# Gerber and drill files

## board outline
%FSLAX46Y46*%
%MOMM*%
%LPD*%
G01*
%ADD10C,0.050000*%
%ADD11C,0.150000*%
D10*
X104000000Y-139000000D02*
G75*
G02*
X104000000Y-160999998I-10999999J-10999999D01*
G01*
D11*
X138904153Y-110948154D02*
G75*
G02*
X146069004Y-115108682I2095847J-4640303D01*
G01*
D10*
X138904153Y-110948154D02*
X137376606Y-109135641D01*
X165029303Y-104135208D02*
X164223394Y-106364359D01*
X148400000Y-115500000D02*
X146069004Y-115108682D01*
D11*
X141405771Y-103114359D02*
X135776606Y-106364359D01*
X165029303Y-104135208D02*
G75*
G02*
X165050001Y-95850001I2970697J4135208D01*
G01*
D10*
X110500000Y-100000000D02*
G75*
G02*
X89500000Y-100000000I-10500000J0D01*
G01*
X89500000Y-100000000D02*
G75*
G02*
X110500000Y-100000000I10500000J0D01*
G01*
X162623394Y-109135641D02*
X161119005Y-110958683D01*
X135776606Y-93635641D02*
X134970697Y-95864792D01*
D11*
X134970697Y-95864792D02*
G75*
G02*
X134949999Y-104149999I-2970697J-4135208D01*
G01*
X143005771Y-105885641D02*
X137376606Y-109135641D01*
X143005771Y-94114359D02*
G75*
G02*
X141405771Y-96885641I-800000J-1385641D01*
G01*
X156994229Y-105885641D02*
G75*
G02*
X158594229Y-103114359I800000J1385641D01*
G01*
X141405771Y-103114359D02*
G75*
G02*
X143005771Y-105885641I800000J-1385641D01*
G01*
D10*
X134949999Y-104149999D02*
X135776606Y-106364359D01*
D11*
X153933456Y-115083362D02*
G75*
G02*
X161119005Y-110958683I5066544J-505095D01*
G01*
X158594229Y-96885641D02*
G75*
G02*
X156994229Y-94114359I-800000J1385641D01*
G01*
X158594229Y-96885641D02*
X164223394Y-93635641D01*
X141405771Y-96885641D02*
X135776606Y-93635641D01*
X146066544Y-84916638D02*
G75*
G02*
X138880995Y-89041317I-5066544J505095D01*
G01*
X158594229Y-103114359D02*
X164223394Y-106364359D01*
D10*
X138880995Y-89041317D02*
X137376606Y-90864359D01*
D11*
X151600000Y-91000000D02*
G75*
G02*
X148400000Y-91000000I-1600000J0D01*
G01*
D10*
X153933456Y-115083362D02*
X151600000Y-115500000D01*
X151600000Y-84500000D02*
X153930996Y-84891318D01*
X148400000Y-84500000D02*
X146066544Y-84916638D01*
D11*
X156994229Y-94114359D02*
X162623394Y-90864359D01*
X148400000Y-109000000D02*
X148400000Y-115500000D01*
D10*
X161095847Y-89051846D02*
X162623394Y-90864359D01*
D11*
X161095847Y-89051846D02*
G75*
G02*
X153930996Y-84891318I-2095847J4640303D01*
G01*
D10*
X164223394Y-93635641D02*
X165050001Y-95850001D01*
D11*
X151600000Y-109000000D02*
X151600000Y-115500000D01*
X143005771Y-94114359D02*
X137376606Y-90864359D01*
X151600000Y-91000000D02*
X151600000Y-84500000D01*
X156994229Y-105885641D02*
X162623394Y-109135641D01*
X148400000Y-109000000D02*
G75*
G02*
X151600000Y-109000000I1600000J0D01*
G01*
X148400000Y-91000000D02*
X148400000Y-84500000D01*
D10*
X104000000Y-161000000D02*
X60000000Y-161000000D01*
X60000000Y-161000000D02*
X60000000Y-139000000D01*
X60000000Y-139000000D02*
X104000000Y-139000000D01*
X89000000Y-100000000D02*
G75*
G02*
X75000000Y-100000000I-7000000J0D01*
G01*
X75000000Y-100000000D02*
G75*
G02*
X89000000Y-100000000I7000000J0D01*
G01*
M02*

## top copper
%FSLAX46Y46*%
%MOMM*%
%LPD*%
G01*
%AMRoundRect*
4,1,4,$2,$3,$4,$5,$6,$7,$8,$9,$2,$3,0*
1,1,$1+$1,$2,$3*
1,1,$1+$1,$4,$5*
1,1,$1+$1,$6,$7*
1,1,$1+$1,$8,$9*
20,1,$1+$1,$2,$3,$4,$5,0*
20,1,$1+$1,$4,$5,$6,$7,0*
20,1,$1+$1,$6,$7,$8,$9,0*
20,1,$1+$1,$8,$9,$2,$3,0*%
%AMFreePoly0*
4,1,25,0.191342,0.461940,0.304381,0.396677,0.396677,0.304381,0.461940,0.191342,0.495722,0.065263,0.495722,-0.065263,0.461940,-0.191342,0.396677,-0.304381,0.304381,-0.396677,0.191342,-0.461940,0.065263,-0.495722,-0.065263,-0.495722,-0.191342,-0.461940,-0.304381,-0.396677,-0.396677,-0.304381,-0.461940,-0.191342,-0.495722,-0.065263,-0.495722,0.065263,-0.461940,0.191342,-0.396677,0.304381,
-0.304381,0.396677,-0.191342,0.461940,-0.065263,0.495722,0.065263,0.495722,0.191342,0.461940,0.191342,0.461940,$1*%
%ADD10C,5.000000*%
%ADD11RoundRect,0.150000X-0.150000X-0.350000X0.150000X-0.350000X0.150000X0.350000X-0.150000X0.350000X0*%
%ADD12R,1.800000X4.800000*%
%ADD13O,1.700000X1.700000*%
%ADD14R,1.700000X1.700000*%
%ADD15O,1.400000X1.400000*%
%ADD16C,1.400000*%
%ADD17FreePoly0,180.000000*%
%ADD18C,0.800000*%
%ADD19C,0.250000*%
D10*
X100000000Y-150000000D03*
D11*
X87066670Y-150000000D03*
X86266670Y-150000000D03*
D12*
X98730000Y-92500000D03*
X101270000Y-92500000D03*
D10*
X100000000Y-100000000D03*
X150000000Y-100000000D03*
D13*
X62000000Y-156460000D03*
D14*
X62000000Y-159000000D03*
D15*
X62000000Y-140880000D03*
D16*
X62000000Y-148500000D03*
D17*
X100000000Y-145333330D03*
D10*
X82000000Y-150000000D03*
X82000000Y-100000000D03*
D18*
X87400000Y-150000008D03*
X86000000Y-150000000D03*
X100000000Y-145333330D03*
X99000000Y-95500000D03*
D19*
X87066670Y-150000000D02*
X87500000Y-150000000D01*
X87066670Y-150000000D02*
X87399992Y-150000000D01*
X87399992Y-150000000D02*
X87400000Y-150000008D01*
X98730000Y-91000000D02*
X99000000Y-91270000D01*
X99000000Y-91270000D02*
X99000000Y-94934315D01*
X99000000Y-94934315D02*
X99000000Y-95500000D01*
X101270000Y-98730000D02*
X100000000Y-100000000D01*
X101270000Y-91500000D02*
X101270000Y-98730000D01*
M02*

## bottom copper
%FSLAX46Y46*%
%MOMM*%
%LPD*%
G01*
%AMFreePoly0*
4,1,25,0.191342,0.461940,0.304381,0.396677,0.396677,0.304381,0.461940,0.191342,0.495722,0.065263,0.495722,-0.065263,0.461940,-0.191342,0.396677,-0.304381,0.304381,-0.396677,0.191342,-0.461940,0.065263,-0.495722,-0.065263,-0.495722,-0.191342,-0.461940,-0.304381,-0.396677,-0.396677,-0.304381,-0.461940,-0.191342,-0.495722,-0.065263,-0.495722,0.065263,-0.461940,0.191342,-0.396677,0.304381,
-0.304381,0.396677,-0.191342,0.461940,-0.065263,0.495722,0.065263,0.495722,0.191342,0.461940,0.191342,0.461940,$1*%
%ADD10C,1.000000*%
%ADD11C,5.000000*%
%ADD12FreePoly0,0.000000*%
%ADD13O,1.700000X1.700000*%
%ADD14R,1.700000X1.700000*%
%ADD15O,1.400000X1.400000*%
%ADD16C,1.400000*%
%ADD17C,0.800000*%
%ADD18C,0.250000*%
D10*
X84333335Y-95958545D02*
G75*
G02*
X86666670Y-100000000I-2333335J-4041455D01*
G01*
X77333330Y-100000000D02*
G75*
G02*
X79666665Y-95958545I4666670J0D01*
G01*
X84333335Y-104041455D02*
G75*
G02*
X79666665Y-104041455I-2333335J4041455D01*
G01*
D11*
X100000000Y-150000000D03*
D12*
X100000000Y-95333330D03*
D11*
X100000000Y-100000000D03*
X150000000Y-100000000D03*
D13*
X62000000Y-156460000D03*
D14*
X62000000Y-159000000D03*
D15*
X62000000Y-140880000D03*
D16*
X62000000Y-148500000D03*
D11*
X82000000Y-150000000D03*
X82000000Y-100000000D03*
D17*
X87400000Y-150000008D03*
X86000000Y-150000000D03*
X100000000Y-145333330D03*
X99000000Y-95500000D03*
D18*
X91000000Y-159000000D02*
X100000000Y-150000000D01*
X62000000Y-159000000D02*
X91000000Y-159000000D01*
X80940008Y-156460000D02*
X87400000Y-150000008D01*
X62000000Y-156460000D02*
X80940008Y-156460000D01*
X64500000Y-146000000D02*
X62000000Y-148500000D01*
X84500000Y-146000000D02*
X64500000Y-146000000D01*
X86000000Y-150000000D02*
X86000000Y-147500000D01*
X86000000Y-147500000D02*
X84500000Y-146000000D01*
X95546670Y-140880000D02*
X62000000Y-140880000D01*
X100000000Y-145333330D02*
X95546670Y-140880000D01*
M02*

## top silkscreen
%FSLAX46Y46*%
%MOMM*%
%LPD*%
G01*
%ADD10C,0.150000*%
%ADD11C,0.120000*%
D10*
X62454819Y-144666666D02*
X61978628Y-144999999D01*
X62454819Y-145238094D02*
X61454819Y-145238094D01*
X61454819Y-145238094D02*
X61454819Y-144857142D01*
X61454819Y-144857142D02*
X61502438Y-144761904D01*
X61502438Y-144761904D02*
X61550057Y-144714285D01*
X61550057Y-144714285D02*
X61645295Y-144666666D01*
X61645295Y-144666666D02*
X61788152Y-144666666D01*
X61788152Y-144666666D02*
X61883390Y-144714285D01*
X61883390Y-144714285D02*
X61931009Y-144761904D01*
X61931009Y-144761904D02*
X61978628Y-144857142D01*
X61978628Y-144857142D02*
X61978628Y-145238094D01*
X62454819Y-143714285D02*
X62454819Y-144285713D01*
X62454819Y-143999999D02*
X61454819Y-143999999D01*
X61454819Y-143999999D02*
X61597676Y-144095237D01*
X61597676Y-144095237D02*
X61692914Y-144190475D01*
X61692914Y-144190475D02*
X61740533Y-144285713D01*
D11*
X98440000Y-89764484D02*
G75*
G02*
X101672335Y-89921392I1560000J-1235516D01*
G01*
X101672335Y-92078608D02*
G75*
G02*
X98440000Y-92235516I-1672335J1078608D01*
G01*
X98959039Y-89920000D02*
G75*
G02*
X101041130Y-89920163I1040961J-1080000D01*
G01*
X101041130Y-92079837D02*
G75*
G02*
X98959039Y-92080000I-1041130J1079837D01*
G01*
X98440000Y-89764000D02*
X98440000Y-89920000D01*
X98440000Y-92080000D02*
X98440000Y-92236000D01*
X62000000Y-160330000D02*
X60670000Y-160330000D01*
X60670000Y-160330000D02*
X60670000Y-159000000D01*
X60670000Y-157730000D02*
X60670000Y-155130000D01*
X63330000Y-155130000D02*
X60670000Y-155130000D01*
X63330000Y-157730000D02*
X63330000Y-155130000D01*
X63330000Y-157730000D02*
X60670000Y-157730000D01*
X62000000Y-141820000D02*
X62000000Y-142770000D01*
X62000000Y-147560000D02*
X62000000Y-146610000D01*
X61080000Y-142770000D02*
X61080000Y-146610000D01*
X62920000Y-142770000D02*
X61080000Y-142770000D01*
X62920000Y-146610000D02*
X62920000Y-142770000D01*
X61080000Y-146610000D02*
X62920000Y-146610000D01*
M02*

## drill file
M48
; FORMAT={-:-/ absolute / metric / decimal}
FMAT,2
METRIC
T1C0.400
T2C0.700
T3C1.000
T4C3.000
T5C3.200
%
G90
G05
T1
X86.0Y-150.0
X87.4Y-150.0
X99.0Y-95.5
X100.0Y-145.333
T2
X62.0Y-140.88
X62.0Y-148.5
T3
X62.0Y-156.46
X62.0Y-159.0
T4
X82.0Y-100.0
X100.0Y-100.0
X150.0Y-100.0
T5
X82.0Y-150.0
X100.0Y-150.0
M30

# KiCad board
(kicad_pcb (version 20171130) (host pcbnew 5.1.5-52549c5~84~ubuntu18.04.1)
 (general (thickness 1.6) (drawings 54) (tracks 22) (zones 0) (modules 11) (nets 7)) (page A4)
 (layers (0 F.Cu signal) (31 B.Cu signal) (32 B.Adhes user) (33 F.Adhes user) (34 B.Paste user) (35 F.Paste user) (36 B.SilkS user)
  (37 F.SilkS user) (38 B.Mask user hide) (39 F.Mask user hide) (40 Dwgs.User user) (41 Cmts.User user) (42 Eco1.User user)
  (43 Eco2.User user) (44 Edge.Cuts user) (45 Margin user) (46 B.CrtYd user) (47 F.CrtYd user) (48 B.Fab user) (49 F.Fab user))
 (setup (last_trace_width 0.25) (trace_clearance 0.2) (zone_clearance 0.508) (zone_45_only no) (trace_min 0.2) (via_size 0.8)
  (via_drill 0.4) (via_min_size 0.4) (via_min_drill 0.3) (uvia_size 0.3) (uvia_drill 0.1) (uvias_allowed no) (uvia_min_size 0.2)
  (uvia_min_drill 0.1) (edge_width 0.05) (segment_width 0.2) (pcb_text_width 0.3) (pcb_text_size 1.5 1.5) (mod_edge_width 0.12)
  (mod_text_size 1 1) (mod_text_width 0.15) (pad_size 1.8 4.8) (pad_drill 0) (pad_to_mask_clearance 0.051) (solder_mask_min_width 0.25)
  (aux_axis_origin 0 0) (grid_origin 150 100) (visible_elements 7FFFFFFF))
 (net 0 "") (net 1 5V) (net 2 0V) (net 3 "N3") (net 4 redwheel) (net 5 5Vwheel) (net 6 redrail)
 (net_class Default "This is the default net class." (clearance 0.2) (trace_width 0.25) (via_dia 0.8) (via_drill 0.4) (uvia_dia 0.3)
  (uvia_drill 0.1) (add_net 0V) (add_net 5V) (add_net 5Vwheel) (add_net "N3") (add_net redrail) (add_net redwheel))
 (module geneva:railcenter (layer F.Cu) (at 100 150)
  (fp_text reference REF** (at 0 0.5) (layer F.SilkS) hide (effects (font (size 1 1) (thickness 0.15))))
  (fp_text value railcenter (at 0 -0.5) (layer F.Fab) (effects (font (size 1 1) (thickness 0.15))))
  (pad 1 thru_hole circle (at 0 0) (size 5 5) (drill 3.2) (layers *.Cu *.Mask) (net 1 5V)))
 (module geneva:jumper (layer F.Cu) (at 86.66667 150)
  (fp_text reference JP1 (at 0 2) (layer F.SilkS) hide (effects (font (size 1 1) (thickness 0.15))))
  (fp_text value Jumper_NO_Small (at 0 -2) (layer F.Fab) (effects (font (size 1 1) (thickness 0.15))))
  (pad 2 smd roundrect (at 0.4 0) (size 0.6 1) (layers F.Cu F.Mask) (roundrect_rratio 0.25) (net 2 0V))
  (pad 1 smd roundrect (at -0.4 0) (size 0.6 1) (layers F.Cu F.Mask) (roundrect_rratio 0.25) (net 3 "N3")))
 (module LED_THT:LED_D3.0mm (layer F.Cu) (at 100 91)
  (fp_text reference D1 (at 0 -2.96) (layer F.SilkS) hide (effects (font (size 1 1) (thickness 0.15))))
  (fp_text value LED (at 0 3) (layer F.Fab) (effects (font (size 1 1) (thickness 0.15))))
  (fp_arc (start 0 0) (end -1.56 -1.235516) (angle 108.8) (layer F.SilkS) (width 0.12))
  (fp_arc (start 0 0) (end -1.56 1.235516) (angle -108.8) (layer F.SilkS) (width 0.12))
  (fp_arc (start 0 0) (end -1.040961 -1.08) (angle 87.9) (layer F.SilkS) (width 0.12))
  (fp_arc (start 0 0) (end -1.040961 1.08) (angle -87.9) (layer F.SilkS) (width 0.12))
  (fp_line (start -1.56 -1.236) (end -1.56 -1.08) (layer F.SilkS) (width 0.12))
  (fp_line (start -1.56 1.08) (end -1.56 1.236) (layer F.SilkS) (width 0.12))
  (pad 1 smd rect (at -1.27 1.5) (size 1.8 4.8) (layers F.Cu F.Paste F.Mask) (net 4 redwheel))
  (pad 2 smd rect (at 1.27 1.5) (size 1.8 4.8) (layers F.Cu F.Paste F.Mask) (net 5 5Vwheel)))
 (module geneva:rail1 (layer B.Cu) (at 100 100)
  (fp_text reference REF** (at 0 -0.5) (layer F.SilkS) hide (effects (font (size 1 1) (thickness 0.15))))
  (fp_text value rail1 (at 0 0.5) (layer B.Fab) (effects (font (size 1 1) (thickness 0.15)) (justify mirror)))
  (pad 1 smd custom (at 0 -4.66667) (size 1 1) (layers B.Cu B.Mask) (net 4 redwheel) (zone_connect 0)
   (options (clearance outline) (anchor circle)) (primitives)))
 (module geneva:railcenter (layer F.Cu) (at 100 100)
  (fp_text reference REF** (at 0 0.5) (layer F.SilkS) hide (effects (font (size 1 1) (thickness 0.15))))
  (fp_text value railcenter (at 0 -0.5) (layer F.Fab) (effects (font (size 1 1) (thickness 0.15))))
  (pad 1 thru_hole circle (at 0 0) (size 5 5) (drill 3) (layers *.Cu *.Mask) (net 5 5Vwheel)))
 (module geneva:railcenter (layer F.Cu) (at 150 100)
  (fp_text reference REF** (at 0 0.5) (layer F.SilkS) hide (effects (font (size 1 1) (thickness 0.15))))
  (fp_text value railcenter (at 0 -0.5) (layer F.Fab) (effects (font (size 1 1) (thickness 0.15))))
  (pad 1 thru_hole circle (at 0 0) (size 5 5) (drill 3) (layers *.Cu *.Mask)))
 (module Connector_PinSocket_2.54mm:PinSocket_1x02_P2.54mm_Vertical (layer F.Cu) (at 62 159 180)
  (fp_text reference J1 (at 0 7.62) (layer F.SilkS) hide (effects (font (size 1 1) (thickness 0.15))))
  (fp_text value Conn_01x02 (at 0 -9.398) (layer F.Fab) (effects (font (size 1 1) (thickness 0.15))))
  (fp_line (start 0 -1.33) (end 1.33 -1.33) (layer F.SilkS) (width 0.12))
  (fp_line (start 1.33 -1.33) (end 1.33 0) (layer F.SilkS) (width 0.12))
  (fp_line (start 1.33 1.27) (end 1.33 3.87) (layer F.SilkS) (width 0.12))
  (fp_line (start -1.33 3.87) (end 1.33 3.87) (layer F.SilkS) (width 0.12))
  (fp_line (start -1.33 1.27) (end -1.33 3.87) (layer F.SilkS) (width 0.12))
  (fp_line (start -1.33 1.27) (end 1.33 1.27) (layer F.SilkS) (width 0.12))
  (pad 2 thru_hole oval (at 0 2.54 180) (size 1.7 1.7) (drill 1) (layers *.Cu *.Mask) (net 2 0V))
  (pad 1 thru_hole rect (at 0 0 180) (size 1.7 1.7) (drill 1) (layers *.Cu *.Mask) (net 1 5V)))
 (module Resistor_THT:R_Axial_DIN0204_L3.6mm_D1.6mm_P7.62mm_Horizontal (layer F.Cu) (at 62 148.5 90)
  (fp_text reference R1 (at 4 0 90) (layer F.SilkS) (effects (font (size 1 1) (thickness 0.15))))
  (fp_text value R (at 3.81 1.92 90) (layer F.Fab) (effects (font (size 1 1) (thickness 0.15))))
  (fp_line (start 6.68 0) (end 5.73 0) (layer F.SilkS) (width 0.12))
  (fp_line (start 0.94 0) (end 1.89 0) (layer F.SilkS) (width 0.12))
  (fp_line (start 5.73 -0.92) (end 1.89 -0.92) (layer F.SilkS) (width 0.12))
  (fp_line (start 5.73 0.92) (end 5.73 -0.92) (layer F.SilkS) (width 0.12))
  (fp_line (start 1.89 0.92) (end 5.73 0.92) (layer F.SilkS) (width 0.12))
  (fp_line (start 1.89 -0.92) (end 1.89 0.92) (layer F.SilkS) (width 0.12))
  (pad 2 thru_hole oval (at 7.62 0 90) (size 1.4 1.4) (drill 0.7) (layers *.Cu *.Mask) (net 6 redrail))
  (pad 1 thru_hole circle (at 0 0 90) (size 1.4 1.4) (drill 0.7) (layers *.Cu *.Mask) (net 3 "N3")))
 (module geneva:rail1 (layer F.Cu) (at 100 150 180)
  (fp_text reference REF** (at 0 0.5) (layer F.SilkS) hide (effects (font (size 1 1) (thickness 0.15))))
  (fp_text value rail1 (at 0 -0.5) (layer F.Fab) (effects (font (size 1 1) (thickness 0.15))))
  (pad 1 smd custom (at 0 4.66667 180) (size 1 1) (layers F.Cu F.Mask) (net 6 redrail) (zone_connect 0)
   (options (clearance outline) (anchor circle)) (primitives)))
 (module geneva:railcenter (layer F.Cu) (at 82 150)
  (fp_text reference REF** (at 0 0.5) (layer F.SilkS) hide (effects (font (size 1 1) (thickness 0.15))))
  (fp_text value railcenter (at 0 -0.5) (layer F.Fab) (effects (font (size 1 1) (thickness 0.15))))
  (pad 1 thru_hole circle (at 0 0) (size 5 5) (drill 3.2) (layers *.Cu *.Mask)))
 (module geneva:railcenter (layer F.Cu) (at 82 100)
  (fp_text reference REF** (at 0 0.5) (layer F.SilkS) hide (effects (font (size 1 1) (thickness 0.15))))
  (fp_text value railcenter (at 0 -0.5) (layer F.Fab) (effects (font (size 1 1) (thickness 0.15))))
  (pad 1 thru_hole circle (at 0 0) (size 5 5) (drill 3) (layers *.Cu *.Mask)))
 (gr_arc (start 93.000001 149.999999) (end 104 160.999998) (angle -90) (layer Edge.Cuts) (width 0.05))
 (gr_arc (start 141 115.588457) (end 146.069004 115.108682) (angle -108.9) (layer Edge.Cuts) (width 0.15))
 (gr_line (start 138.904153 110.948154) (end 137.376606 109.135641) (layer Edge.Cuts) (width 0.05))
 (gr_line (start 165.029303 104.135208) (end 164.223394 106.364359) (layer Edge.Cuts) (width 0.05))
 (gr_line (start 148.4 115.5) (end 146.069004 115.108682) (layer Edge.Cuts) (width 0.05))
 (gr_line (start 141.405771 103.114359) (end 135.776606 106.364359) (layer Edge.Cuts) (width 0.15))
 (gr_arc (start 168 100) (end 165.050001 95.850001) (angle -108.9) (layer Edge.Cuts) (width 0.15))
 (gr_circle (center 100 100) (end 110.5 100) (layer Edge.Cuts) (width 0.05))
 (gr_line (start 162.623394 109.135641) (end 161.119005 110.958683) (layer Edge.Cuts) (width 0.05))
 (gr_line (start 135.776606 93.635641) (end 134.970697 95.864792) (layer Edge.Cuts) (width 0.05))
 (gr_arc (start 132 100) (end 134.949999 104.149999) (angle -108.9) (layer Edge.Cuts) (width 0.15))
 (gr_line (start 143.005771 105.885641) (end 137.376606 109.135641) (layer Edge.Cuts) (width 0.15))
 (gr_arc (start 142.205771 95.5) (end 141.405771 96.885641) (angle -180) (layer Edge.Cuts) (width 0.15))
 (gr_arc (start 157.794229 104.5) (end 158.594229 103.114359) (angle -180) (layer Edge.Cuts) (width 0.15))
 (gr_arc (start 142.205771 104.5) (end 143.005771 105.885641) (angle -180) (layer Edge.Cuts) (width 0.15))
 (gr_line (start 134.949999 104.149999) (end 135.776606 106.364359) (layer Edge.Cuts) (width 0.05))
 (gr_arc (start 159 115.588457) (end 161.119005 110.958683) (angle -108.9) (layer Edge.Cuts) (width 0.15))
 (gr_arc (start 157.794229 95.5) (end 156.994229 94.114359) (angle -180) (layer Edge.Cuts) (width 0.15))
 (gr_line (start 158.594229 96.885641) (end 164.223394 93.635641) (layer Edge.Cuts) (width 0.15))
 (gr_line (start 141.405771 96.885641) (end 135.776606 93.635641) (layer Edge.Cuts) (width 0.15))
 (gr_arc (start 141 84.411543) (end 138.880995 89.041317) (angle -108.9) (layer Edge.Cuts) (width 0.15))
 (gr_line (start 158.594229 103.114359) (end 164.223394 106.364359) (layer Edge.Cuts) (width 0.15))
 (gr_line (start 138.880995 89.041317) (end 137.376606 90.864359) (layer Edge.Cuts) (width 0.05))
 (gr_arc (start 150 91) (end 148.4 91) (angle -180) (layer Edge.Cuts) (width 0.15))
 (gr_line (start 153.933456 115.083362) (end 151.6 115.5) (layer Edge.Cuts) (width 0.05))
 (gr_line (start 151.6 84.5) (end 153.930996 84.891318) (layer Edge.Cuts) (width 0.05))
 (gr_line (start 148.4 84.5) (end 146.066544 84.916638) (layer Edge.Cuts) (width 0.05))
 (gr_line (start 156.994229 94.114359) (end 162.623394 90.864359) (layer Edge.Cuts) (width 0.15))
 (gr_line (start 148.4 109) (end 148.4 115.5) (layer Edge.Cuts) (width 0.15))
 (gr_line (start 161.095847 89.051846) (end 162.623394 90.864359) (layer Edge.Cuts) (width 0.05))
 (gr_arc (start 159 84.411543) (end 153.930996 84.891318) (angle -108.9) (layer Edge.Cuts) (width 0.15))
 (gr_line (start 164.223394 93.635641) (end 165.050001 95.850001) (layer Edge.Cuts) (width 0.05))
 (gr_line (start 151.6 109) (end 151.6 115.5) (layer Edge.Cuts) (width 0.15))
 (gr_line (start 143.005771 94.114359) (end 137.376606 90.864359) (layer Edge.Cuts) (width 0.15))
 (gr_line (start 151.6 91) (end 151.6 84.5) (layer Edge.Cuts) (width 0.15))
 (gr_line (start 156.994229 105.885641) (end 162.623394 109.135641) (layer Edge.Cuts) (width 0.15))
 (gr_arc (start 150 109) (end 151.6 109) (angle -180) (layer Edge.Cuts) (width 0.15))
 (gr_line (start 148.4 91) (end 148.4 84.5) (layer Edge.Cuts) (width 0.15))
 (gr_line (start 104 161) (end 60 161) (layer Edge.Cuts) (width 0.05))
 (gr_line (start 60 161) (end 60 139) (layer Edge.Cuts) (width 0.05))
 (gr_line (start 60 139) (end 104 139) (layer Edge.Cuts) (width 0.05))
 (gr_circle (center 82 100) (end 89 100) (layer Edge.Cuts) (width 0.05))
 (gr_arc (start 82 100) (end 86.66667 100) (angle -60) (layer B.Cu) (width 1))
 (gr_arc (start 82 100) (end 79.666665 95.958545) (angle -60) (layer B.Cu) (width 1))
 (gr_arc (start 82 100) (end 79.666665 104.041455) (angle -60) (layer B.Cu) (width 1))
 (segment (start 91 159) (end 100 150) (width 0.25) (layer B.Cu) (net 1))
 (segment (start 62 159) (end 91 159) (width 0.25) (layer B.Cu) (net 1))
 (segment (start 87.06667 150) (end 87.5 150) (width 0.25) (layer F.Cu) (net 2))
 (segment (start 87.06667 150) (end 87.399992 150) (width 0.25) (layer F.Cu) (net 2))
 (segment (start 87.399992 150) (end 87.4 150.000008) (width 0.25) (layer F.Cu) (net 2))
 (via (at 87.4 150.000008) (size 0.8) (drill 0.4) (layers F.Cu B.Cu) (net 2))
 (segment (start 80.940008 156.46) (end 87.4 150.000008) (width 0.25) (layer B.Cu) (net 2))
 (segment (start 62 156.46) (end 80.940008 156.46) (width 0.25) (layer B.Cu) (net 2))
 (via (at 86 150) (size 0.8) (drill 0.4) (layers F.Cu B.Cu) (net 3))
 (segment (start 64.5 146) (end 62 148.5) (width 0.25) (layer B.Cu) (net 3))
 (segment (start 84.5 146) (end 64.5 146) (width 0.25) (layer B.Cu) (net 3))
 (segment (start 86 150) (end 86 147.5) (width 0.25) (layer B.Cu) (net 3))
 (segment (start 86 147.5) (end 84.5 146) (width 0.25) (layer B.Cu) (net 3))
 (via (at 100 145.33333) (size 0.8) (drill 0.4) (layers F.Cu B.Cu) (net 6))
 (segment (start 95.54667 140.88) (end 62 140.88) (width 0.25) (layer B.Cu) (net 6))
 (segment (start 100 145.33333) (end 95.54667 140.88) (width 0.25) (layer B.Cu) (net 6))
 (segment (start 98.73 91) (end 99 91.27) (width 0.25) (layer F.Cu) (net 4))
 (segment (start 99 91.27) (end 99 94.934315) (width 0.25) (layer F.Cu) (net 4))
 (segment (start 99 94.934315) (end 99 95.5) (width 0.25) (layer F.Cu) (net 4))
 (via (at 99 95.5) (size 0.8) (drill 0.4) (layers F.Cu B.Cu) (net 4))
 (segment (start 101.27 98.73) (end 100 100) (width 0.25) (layer F.Cu) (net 5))
 (segment (start 101.27 91.5) (end 101.27 98.73) (width 0.25) (layer F.Cu) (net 5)))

